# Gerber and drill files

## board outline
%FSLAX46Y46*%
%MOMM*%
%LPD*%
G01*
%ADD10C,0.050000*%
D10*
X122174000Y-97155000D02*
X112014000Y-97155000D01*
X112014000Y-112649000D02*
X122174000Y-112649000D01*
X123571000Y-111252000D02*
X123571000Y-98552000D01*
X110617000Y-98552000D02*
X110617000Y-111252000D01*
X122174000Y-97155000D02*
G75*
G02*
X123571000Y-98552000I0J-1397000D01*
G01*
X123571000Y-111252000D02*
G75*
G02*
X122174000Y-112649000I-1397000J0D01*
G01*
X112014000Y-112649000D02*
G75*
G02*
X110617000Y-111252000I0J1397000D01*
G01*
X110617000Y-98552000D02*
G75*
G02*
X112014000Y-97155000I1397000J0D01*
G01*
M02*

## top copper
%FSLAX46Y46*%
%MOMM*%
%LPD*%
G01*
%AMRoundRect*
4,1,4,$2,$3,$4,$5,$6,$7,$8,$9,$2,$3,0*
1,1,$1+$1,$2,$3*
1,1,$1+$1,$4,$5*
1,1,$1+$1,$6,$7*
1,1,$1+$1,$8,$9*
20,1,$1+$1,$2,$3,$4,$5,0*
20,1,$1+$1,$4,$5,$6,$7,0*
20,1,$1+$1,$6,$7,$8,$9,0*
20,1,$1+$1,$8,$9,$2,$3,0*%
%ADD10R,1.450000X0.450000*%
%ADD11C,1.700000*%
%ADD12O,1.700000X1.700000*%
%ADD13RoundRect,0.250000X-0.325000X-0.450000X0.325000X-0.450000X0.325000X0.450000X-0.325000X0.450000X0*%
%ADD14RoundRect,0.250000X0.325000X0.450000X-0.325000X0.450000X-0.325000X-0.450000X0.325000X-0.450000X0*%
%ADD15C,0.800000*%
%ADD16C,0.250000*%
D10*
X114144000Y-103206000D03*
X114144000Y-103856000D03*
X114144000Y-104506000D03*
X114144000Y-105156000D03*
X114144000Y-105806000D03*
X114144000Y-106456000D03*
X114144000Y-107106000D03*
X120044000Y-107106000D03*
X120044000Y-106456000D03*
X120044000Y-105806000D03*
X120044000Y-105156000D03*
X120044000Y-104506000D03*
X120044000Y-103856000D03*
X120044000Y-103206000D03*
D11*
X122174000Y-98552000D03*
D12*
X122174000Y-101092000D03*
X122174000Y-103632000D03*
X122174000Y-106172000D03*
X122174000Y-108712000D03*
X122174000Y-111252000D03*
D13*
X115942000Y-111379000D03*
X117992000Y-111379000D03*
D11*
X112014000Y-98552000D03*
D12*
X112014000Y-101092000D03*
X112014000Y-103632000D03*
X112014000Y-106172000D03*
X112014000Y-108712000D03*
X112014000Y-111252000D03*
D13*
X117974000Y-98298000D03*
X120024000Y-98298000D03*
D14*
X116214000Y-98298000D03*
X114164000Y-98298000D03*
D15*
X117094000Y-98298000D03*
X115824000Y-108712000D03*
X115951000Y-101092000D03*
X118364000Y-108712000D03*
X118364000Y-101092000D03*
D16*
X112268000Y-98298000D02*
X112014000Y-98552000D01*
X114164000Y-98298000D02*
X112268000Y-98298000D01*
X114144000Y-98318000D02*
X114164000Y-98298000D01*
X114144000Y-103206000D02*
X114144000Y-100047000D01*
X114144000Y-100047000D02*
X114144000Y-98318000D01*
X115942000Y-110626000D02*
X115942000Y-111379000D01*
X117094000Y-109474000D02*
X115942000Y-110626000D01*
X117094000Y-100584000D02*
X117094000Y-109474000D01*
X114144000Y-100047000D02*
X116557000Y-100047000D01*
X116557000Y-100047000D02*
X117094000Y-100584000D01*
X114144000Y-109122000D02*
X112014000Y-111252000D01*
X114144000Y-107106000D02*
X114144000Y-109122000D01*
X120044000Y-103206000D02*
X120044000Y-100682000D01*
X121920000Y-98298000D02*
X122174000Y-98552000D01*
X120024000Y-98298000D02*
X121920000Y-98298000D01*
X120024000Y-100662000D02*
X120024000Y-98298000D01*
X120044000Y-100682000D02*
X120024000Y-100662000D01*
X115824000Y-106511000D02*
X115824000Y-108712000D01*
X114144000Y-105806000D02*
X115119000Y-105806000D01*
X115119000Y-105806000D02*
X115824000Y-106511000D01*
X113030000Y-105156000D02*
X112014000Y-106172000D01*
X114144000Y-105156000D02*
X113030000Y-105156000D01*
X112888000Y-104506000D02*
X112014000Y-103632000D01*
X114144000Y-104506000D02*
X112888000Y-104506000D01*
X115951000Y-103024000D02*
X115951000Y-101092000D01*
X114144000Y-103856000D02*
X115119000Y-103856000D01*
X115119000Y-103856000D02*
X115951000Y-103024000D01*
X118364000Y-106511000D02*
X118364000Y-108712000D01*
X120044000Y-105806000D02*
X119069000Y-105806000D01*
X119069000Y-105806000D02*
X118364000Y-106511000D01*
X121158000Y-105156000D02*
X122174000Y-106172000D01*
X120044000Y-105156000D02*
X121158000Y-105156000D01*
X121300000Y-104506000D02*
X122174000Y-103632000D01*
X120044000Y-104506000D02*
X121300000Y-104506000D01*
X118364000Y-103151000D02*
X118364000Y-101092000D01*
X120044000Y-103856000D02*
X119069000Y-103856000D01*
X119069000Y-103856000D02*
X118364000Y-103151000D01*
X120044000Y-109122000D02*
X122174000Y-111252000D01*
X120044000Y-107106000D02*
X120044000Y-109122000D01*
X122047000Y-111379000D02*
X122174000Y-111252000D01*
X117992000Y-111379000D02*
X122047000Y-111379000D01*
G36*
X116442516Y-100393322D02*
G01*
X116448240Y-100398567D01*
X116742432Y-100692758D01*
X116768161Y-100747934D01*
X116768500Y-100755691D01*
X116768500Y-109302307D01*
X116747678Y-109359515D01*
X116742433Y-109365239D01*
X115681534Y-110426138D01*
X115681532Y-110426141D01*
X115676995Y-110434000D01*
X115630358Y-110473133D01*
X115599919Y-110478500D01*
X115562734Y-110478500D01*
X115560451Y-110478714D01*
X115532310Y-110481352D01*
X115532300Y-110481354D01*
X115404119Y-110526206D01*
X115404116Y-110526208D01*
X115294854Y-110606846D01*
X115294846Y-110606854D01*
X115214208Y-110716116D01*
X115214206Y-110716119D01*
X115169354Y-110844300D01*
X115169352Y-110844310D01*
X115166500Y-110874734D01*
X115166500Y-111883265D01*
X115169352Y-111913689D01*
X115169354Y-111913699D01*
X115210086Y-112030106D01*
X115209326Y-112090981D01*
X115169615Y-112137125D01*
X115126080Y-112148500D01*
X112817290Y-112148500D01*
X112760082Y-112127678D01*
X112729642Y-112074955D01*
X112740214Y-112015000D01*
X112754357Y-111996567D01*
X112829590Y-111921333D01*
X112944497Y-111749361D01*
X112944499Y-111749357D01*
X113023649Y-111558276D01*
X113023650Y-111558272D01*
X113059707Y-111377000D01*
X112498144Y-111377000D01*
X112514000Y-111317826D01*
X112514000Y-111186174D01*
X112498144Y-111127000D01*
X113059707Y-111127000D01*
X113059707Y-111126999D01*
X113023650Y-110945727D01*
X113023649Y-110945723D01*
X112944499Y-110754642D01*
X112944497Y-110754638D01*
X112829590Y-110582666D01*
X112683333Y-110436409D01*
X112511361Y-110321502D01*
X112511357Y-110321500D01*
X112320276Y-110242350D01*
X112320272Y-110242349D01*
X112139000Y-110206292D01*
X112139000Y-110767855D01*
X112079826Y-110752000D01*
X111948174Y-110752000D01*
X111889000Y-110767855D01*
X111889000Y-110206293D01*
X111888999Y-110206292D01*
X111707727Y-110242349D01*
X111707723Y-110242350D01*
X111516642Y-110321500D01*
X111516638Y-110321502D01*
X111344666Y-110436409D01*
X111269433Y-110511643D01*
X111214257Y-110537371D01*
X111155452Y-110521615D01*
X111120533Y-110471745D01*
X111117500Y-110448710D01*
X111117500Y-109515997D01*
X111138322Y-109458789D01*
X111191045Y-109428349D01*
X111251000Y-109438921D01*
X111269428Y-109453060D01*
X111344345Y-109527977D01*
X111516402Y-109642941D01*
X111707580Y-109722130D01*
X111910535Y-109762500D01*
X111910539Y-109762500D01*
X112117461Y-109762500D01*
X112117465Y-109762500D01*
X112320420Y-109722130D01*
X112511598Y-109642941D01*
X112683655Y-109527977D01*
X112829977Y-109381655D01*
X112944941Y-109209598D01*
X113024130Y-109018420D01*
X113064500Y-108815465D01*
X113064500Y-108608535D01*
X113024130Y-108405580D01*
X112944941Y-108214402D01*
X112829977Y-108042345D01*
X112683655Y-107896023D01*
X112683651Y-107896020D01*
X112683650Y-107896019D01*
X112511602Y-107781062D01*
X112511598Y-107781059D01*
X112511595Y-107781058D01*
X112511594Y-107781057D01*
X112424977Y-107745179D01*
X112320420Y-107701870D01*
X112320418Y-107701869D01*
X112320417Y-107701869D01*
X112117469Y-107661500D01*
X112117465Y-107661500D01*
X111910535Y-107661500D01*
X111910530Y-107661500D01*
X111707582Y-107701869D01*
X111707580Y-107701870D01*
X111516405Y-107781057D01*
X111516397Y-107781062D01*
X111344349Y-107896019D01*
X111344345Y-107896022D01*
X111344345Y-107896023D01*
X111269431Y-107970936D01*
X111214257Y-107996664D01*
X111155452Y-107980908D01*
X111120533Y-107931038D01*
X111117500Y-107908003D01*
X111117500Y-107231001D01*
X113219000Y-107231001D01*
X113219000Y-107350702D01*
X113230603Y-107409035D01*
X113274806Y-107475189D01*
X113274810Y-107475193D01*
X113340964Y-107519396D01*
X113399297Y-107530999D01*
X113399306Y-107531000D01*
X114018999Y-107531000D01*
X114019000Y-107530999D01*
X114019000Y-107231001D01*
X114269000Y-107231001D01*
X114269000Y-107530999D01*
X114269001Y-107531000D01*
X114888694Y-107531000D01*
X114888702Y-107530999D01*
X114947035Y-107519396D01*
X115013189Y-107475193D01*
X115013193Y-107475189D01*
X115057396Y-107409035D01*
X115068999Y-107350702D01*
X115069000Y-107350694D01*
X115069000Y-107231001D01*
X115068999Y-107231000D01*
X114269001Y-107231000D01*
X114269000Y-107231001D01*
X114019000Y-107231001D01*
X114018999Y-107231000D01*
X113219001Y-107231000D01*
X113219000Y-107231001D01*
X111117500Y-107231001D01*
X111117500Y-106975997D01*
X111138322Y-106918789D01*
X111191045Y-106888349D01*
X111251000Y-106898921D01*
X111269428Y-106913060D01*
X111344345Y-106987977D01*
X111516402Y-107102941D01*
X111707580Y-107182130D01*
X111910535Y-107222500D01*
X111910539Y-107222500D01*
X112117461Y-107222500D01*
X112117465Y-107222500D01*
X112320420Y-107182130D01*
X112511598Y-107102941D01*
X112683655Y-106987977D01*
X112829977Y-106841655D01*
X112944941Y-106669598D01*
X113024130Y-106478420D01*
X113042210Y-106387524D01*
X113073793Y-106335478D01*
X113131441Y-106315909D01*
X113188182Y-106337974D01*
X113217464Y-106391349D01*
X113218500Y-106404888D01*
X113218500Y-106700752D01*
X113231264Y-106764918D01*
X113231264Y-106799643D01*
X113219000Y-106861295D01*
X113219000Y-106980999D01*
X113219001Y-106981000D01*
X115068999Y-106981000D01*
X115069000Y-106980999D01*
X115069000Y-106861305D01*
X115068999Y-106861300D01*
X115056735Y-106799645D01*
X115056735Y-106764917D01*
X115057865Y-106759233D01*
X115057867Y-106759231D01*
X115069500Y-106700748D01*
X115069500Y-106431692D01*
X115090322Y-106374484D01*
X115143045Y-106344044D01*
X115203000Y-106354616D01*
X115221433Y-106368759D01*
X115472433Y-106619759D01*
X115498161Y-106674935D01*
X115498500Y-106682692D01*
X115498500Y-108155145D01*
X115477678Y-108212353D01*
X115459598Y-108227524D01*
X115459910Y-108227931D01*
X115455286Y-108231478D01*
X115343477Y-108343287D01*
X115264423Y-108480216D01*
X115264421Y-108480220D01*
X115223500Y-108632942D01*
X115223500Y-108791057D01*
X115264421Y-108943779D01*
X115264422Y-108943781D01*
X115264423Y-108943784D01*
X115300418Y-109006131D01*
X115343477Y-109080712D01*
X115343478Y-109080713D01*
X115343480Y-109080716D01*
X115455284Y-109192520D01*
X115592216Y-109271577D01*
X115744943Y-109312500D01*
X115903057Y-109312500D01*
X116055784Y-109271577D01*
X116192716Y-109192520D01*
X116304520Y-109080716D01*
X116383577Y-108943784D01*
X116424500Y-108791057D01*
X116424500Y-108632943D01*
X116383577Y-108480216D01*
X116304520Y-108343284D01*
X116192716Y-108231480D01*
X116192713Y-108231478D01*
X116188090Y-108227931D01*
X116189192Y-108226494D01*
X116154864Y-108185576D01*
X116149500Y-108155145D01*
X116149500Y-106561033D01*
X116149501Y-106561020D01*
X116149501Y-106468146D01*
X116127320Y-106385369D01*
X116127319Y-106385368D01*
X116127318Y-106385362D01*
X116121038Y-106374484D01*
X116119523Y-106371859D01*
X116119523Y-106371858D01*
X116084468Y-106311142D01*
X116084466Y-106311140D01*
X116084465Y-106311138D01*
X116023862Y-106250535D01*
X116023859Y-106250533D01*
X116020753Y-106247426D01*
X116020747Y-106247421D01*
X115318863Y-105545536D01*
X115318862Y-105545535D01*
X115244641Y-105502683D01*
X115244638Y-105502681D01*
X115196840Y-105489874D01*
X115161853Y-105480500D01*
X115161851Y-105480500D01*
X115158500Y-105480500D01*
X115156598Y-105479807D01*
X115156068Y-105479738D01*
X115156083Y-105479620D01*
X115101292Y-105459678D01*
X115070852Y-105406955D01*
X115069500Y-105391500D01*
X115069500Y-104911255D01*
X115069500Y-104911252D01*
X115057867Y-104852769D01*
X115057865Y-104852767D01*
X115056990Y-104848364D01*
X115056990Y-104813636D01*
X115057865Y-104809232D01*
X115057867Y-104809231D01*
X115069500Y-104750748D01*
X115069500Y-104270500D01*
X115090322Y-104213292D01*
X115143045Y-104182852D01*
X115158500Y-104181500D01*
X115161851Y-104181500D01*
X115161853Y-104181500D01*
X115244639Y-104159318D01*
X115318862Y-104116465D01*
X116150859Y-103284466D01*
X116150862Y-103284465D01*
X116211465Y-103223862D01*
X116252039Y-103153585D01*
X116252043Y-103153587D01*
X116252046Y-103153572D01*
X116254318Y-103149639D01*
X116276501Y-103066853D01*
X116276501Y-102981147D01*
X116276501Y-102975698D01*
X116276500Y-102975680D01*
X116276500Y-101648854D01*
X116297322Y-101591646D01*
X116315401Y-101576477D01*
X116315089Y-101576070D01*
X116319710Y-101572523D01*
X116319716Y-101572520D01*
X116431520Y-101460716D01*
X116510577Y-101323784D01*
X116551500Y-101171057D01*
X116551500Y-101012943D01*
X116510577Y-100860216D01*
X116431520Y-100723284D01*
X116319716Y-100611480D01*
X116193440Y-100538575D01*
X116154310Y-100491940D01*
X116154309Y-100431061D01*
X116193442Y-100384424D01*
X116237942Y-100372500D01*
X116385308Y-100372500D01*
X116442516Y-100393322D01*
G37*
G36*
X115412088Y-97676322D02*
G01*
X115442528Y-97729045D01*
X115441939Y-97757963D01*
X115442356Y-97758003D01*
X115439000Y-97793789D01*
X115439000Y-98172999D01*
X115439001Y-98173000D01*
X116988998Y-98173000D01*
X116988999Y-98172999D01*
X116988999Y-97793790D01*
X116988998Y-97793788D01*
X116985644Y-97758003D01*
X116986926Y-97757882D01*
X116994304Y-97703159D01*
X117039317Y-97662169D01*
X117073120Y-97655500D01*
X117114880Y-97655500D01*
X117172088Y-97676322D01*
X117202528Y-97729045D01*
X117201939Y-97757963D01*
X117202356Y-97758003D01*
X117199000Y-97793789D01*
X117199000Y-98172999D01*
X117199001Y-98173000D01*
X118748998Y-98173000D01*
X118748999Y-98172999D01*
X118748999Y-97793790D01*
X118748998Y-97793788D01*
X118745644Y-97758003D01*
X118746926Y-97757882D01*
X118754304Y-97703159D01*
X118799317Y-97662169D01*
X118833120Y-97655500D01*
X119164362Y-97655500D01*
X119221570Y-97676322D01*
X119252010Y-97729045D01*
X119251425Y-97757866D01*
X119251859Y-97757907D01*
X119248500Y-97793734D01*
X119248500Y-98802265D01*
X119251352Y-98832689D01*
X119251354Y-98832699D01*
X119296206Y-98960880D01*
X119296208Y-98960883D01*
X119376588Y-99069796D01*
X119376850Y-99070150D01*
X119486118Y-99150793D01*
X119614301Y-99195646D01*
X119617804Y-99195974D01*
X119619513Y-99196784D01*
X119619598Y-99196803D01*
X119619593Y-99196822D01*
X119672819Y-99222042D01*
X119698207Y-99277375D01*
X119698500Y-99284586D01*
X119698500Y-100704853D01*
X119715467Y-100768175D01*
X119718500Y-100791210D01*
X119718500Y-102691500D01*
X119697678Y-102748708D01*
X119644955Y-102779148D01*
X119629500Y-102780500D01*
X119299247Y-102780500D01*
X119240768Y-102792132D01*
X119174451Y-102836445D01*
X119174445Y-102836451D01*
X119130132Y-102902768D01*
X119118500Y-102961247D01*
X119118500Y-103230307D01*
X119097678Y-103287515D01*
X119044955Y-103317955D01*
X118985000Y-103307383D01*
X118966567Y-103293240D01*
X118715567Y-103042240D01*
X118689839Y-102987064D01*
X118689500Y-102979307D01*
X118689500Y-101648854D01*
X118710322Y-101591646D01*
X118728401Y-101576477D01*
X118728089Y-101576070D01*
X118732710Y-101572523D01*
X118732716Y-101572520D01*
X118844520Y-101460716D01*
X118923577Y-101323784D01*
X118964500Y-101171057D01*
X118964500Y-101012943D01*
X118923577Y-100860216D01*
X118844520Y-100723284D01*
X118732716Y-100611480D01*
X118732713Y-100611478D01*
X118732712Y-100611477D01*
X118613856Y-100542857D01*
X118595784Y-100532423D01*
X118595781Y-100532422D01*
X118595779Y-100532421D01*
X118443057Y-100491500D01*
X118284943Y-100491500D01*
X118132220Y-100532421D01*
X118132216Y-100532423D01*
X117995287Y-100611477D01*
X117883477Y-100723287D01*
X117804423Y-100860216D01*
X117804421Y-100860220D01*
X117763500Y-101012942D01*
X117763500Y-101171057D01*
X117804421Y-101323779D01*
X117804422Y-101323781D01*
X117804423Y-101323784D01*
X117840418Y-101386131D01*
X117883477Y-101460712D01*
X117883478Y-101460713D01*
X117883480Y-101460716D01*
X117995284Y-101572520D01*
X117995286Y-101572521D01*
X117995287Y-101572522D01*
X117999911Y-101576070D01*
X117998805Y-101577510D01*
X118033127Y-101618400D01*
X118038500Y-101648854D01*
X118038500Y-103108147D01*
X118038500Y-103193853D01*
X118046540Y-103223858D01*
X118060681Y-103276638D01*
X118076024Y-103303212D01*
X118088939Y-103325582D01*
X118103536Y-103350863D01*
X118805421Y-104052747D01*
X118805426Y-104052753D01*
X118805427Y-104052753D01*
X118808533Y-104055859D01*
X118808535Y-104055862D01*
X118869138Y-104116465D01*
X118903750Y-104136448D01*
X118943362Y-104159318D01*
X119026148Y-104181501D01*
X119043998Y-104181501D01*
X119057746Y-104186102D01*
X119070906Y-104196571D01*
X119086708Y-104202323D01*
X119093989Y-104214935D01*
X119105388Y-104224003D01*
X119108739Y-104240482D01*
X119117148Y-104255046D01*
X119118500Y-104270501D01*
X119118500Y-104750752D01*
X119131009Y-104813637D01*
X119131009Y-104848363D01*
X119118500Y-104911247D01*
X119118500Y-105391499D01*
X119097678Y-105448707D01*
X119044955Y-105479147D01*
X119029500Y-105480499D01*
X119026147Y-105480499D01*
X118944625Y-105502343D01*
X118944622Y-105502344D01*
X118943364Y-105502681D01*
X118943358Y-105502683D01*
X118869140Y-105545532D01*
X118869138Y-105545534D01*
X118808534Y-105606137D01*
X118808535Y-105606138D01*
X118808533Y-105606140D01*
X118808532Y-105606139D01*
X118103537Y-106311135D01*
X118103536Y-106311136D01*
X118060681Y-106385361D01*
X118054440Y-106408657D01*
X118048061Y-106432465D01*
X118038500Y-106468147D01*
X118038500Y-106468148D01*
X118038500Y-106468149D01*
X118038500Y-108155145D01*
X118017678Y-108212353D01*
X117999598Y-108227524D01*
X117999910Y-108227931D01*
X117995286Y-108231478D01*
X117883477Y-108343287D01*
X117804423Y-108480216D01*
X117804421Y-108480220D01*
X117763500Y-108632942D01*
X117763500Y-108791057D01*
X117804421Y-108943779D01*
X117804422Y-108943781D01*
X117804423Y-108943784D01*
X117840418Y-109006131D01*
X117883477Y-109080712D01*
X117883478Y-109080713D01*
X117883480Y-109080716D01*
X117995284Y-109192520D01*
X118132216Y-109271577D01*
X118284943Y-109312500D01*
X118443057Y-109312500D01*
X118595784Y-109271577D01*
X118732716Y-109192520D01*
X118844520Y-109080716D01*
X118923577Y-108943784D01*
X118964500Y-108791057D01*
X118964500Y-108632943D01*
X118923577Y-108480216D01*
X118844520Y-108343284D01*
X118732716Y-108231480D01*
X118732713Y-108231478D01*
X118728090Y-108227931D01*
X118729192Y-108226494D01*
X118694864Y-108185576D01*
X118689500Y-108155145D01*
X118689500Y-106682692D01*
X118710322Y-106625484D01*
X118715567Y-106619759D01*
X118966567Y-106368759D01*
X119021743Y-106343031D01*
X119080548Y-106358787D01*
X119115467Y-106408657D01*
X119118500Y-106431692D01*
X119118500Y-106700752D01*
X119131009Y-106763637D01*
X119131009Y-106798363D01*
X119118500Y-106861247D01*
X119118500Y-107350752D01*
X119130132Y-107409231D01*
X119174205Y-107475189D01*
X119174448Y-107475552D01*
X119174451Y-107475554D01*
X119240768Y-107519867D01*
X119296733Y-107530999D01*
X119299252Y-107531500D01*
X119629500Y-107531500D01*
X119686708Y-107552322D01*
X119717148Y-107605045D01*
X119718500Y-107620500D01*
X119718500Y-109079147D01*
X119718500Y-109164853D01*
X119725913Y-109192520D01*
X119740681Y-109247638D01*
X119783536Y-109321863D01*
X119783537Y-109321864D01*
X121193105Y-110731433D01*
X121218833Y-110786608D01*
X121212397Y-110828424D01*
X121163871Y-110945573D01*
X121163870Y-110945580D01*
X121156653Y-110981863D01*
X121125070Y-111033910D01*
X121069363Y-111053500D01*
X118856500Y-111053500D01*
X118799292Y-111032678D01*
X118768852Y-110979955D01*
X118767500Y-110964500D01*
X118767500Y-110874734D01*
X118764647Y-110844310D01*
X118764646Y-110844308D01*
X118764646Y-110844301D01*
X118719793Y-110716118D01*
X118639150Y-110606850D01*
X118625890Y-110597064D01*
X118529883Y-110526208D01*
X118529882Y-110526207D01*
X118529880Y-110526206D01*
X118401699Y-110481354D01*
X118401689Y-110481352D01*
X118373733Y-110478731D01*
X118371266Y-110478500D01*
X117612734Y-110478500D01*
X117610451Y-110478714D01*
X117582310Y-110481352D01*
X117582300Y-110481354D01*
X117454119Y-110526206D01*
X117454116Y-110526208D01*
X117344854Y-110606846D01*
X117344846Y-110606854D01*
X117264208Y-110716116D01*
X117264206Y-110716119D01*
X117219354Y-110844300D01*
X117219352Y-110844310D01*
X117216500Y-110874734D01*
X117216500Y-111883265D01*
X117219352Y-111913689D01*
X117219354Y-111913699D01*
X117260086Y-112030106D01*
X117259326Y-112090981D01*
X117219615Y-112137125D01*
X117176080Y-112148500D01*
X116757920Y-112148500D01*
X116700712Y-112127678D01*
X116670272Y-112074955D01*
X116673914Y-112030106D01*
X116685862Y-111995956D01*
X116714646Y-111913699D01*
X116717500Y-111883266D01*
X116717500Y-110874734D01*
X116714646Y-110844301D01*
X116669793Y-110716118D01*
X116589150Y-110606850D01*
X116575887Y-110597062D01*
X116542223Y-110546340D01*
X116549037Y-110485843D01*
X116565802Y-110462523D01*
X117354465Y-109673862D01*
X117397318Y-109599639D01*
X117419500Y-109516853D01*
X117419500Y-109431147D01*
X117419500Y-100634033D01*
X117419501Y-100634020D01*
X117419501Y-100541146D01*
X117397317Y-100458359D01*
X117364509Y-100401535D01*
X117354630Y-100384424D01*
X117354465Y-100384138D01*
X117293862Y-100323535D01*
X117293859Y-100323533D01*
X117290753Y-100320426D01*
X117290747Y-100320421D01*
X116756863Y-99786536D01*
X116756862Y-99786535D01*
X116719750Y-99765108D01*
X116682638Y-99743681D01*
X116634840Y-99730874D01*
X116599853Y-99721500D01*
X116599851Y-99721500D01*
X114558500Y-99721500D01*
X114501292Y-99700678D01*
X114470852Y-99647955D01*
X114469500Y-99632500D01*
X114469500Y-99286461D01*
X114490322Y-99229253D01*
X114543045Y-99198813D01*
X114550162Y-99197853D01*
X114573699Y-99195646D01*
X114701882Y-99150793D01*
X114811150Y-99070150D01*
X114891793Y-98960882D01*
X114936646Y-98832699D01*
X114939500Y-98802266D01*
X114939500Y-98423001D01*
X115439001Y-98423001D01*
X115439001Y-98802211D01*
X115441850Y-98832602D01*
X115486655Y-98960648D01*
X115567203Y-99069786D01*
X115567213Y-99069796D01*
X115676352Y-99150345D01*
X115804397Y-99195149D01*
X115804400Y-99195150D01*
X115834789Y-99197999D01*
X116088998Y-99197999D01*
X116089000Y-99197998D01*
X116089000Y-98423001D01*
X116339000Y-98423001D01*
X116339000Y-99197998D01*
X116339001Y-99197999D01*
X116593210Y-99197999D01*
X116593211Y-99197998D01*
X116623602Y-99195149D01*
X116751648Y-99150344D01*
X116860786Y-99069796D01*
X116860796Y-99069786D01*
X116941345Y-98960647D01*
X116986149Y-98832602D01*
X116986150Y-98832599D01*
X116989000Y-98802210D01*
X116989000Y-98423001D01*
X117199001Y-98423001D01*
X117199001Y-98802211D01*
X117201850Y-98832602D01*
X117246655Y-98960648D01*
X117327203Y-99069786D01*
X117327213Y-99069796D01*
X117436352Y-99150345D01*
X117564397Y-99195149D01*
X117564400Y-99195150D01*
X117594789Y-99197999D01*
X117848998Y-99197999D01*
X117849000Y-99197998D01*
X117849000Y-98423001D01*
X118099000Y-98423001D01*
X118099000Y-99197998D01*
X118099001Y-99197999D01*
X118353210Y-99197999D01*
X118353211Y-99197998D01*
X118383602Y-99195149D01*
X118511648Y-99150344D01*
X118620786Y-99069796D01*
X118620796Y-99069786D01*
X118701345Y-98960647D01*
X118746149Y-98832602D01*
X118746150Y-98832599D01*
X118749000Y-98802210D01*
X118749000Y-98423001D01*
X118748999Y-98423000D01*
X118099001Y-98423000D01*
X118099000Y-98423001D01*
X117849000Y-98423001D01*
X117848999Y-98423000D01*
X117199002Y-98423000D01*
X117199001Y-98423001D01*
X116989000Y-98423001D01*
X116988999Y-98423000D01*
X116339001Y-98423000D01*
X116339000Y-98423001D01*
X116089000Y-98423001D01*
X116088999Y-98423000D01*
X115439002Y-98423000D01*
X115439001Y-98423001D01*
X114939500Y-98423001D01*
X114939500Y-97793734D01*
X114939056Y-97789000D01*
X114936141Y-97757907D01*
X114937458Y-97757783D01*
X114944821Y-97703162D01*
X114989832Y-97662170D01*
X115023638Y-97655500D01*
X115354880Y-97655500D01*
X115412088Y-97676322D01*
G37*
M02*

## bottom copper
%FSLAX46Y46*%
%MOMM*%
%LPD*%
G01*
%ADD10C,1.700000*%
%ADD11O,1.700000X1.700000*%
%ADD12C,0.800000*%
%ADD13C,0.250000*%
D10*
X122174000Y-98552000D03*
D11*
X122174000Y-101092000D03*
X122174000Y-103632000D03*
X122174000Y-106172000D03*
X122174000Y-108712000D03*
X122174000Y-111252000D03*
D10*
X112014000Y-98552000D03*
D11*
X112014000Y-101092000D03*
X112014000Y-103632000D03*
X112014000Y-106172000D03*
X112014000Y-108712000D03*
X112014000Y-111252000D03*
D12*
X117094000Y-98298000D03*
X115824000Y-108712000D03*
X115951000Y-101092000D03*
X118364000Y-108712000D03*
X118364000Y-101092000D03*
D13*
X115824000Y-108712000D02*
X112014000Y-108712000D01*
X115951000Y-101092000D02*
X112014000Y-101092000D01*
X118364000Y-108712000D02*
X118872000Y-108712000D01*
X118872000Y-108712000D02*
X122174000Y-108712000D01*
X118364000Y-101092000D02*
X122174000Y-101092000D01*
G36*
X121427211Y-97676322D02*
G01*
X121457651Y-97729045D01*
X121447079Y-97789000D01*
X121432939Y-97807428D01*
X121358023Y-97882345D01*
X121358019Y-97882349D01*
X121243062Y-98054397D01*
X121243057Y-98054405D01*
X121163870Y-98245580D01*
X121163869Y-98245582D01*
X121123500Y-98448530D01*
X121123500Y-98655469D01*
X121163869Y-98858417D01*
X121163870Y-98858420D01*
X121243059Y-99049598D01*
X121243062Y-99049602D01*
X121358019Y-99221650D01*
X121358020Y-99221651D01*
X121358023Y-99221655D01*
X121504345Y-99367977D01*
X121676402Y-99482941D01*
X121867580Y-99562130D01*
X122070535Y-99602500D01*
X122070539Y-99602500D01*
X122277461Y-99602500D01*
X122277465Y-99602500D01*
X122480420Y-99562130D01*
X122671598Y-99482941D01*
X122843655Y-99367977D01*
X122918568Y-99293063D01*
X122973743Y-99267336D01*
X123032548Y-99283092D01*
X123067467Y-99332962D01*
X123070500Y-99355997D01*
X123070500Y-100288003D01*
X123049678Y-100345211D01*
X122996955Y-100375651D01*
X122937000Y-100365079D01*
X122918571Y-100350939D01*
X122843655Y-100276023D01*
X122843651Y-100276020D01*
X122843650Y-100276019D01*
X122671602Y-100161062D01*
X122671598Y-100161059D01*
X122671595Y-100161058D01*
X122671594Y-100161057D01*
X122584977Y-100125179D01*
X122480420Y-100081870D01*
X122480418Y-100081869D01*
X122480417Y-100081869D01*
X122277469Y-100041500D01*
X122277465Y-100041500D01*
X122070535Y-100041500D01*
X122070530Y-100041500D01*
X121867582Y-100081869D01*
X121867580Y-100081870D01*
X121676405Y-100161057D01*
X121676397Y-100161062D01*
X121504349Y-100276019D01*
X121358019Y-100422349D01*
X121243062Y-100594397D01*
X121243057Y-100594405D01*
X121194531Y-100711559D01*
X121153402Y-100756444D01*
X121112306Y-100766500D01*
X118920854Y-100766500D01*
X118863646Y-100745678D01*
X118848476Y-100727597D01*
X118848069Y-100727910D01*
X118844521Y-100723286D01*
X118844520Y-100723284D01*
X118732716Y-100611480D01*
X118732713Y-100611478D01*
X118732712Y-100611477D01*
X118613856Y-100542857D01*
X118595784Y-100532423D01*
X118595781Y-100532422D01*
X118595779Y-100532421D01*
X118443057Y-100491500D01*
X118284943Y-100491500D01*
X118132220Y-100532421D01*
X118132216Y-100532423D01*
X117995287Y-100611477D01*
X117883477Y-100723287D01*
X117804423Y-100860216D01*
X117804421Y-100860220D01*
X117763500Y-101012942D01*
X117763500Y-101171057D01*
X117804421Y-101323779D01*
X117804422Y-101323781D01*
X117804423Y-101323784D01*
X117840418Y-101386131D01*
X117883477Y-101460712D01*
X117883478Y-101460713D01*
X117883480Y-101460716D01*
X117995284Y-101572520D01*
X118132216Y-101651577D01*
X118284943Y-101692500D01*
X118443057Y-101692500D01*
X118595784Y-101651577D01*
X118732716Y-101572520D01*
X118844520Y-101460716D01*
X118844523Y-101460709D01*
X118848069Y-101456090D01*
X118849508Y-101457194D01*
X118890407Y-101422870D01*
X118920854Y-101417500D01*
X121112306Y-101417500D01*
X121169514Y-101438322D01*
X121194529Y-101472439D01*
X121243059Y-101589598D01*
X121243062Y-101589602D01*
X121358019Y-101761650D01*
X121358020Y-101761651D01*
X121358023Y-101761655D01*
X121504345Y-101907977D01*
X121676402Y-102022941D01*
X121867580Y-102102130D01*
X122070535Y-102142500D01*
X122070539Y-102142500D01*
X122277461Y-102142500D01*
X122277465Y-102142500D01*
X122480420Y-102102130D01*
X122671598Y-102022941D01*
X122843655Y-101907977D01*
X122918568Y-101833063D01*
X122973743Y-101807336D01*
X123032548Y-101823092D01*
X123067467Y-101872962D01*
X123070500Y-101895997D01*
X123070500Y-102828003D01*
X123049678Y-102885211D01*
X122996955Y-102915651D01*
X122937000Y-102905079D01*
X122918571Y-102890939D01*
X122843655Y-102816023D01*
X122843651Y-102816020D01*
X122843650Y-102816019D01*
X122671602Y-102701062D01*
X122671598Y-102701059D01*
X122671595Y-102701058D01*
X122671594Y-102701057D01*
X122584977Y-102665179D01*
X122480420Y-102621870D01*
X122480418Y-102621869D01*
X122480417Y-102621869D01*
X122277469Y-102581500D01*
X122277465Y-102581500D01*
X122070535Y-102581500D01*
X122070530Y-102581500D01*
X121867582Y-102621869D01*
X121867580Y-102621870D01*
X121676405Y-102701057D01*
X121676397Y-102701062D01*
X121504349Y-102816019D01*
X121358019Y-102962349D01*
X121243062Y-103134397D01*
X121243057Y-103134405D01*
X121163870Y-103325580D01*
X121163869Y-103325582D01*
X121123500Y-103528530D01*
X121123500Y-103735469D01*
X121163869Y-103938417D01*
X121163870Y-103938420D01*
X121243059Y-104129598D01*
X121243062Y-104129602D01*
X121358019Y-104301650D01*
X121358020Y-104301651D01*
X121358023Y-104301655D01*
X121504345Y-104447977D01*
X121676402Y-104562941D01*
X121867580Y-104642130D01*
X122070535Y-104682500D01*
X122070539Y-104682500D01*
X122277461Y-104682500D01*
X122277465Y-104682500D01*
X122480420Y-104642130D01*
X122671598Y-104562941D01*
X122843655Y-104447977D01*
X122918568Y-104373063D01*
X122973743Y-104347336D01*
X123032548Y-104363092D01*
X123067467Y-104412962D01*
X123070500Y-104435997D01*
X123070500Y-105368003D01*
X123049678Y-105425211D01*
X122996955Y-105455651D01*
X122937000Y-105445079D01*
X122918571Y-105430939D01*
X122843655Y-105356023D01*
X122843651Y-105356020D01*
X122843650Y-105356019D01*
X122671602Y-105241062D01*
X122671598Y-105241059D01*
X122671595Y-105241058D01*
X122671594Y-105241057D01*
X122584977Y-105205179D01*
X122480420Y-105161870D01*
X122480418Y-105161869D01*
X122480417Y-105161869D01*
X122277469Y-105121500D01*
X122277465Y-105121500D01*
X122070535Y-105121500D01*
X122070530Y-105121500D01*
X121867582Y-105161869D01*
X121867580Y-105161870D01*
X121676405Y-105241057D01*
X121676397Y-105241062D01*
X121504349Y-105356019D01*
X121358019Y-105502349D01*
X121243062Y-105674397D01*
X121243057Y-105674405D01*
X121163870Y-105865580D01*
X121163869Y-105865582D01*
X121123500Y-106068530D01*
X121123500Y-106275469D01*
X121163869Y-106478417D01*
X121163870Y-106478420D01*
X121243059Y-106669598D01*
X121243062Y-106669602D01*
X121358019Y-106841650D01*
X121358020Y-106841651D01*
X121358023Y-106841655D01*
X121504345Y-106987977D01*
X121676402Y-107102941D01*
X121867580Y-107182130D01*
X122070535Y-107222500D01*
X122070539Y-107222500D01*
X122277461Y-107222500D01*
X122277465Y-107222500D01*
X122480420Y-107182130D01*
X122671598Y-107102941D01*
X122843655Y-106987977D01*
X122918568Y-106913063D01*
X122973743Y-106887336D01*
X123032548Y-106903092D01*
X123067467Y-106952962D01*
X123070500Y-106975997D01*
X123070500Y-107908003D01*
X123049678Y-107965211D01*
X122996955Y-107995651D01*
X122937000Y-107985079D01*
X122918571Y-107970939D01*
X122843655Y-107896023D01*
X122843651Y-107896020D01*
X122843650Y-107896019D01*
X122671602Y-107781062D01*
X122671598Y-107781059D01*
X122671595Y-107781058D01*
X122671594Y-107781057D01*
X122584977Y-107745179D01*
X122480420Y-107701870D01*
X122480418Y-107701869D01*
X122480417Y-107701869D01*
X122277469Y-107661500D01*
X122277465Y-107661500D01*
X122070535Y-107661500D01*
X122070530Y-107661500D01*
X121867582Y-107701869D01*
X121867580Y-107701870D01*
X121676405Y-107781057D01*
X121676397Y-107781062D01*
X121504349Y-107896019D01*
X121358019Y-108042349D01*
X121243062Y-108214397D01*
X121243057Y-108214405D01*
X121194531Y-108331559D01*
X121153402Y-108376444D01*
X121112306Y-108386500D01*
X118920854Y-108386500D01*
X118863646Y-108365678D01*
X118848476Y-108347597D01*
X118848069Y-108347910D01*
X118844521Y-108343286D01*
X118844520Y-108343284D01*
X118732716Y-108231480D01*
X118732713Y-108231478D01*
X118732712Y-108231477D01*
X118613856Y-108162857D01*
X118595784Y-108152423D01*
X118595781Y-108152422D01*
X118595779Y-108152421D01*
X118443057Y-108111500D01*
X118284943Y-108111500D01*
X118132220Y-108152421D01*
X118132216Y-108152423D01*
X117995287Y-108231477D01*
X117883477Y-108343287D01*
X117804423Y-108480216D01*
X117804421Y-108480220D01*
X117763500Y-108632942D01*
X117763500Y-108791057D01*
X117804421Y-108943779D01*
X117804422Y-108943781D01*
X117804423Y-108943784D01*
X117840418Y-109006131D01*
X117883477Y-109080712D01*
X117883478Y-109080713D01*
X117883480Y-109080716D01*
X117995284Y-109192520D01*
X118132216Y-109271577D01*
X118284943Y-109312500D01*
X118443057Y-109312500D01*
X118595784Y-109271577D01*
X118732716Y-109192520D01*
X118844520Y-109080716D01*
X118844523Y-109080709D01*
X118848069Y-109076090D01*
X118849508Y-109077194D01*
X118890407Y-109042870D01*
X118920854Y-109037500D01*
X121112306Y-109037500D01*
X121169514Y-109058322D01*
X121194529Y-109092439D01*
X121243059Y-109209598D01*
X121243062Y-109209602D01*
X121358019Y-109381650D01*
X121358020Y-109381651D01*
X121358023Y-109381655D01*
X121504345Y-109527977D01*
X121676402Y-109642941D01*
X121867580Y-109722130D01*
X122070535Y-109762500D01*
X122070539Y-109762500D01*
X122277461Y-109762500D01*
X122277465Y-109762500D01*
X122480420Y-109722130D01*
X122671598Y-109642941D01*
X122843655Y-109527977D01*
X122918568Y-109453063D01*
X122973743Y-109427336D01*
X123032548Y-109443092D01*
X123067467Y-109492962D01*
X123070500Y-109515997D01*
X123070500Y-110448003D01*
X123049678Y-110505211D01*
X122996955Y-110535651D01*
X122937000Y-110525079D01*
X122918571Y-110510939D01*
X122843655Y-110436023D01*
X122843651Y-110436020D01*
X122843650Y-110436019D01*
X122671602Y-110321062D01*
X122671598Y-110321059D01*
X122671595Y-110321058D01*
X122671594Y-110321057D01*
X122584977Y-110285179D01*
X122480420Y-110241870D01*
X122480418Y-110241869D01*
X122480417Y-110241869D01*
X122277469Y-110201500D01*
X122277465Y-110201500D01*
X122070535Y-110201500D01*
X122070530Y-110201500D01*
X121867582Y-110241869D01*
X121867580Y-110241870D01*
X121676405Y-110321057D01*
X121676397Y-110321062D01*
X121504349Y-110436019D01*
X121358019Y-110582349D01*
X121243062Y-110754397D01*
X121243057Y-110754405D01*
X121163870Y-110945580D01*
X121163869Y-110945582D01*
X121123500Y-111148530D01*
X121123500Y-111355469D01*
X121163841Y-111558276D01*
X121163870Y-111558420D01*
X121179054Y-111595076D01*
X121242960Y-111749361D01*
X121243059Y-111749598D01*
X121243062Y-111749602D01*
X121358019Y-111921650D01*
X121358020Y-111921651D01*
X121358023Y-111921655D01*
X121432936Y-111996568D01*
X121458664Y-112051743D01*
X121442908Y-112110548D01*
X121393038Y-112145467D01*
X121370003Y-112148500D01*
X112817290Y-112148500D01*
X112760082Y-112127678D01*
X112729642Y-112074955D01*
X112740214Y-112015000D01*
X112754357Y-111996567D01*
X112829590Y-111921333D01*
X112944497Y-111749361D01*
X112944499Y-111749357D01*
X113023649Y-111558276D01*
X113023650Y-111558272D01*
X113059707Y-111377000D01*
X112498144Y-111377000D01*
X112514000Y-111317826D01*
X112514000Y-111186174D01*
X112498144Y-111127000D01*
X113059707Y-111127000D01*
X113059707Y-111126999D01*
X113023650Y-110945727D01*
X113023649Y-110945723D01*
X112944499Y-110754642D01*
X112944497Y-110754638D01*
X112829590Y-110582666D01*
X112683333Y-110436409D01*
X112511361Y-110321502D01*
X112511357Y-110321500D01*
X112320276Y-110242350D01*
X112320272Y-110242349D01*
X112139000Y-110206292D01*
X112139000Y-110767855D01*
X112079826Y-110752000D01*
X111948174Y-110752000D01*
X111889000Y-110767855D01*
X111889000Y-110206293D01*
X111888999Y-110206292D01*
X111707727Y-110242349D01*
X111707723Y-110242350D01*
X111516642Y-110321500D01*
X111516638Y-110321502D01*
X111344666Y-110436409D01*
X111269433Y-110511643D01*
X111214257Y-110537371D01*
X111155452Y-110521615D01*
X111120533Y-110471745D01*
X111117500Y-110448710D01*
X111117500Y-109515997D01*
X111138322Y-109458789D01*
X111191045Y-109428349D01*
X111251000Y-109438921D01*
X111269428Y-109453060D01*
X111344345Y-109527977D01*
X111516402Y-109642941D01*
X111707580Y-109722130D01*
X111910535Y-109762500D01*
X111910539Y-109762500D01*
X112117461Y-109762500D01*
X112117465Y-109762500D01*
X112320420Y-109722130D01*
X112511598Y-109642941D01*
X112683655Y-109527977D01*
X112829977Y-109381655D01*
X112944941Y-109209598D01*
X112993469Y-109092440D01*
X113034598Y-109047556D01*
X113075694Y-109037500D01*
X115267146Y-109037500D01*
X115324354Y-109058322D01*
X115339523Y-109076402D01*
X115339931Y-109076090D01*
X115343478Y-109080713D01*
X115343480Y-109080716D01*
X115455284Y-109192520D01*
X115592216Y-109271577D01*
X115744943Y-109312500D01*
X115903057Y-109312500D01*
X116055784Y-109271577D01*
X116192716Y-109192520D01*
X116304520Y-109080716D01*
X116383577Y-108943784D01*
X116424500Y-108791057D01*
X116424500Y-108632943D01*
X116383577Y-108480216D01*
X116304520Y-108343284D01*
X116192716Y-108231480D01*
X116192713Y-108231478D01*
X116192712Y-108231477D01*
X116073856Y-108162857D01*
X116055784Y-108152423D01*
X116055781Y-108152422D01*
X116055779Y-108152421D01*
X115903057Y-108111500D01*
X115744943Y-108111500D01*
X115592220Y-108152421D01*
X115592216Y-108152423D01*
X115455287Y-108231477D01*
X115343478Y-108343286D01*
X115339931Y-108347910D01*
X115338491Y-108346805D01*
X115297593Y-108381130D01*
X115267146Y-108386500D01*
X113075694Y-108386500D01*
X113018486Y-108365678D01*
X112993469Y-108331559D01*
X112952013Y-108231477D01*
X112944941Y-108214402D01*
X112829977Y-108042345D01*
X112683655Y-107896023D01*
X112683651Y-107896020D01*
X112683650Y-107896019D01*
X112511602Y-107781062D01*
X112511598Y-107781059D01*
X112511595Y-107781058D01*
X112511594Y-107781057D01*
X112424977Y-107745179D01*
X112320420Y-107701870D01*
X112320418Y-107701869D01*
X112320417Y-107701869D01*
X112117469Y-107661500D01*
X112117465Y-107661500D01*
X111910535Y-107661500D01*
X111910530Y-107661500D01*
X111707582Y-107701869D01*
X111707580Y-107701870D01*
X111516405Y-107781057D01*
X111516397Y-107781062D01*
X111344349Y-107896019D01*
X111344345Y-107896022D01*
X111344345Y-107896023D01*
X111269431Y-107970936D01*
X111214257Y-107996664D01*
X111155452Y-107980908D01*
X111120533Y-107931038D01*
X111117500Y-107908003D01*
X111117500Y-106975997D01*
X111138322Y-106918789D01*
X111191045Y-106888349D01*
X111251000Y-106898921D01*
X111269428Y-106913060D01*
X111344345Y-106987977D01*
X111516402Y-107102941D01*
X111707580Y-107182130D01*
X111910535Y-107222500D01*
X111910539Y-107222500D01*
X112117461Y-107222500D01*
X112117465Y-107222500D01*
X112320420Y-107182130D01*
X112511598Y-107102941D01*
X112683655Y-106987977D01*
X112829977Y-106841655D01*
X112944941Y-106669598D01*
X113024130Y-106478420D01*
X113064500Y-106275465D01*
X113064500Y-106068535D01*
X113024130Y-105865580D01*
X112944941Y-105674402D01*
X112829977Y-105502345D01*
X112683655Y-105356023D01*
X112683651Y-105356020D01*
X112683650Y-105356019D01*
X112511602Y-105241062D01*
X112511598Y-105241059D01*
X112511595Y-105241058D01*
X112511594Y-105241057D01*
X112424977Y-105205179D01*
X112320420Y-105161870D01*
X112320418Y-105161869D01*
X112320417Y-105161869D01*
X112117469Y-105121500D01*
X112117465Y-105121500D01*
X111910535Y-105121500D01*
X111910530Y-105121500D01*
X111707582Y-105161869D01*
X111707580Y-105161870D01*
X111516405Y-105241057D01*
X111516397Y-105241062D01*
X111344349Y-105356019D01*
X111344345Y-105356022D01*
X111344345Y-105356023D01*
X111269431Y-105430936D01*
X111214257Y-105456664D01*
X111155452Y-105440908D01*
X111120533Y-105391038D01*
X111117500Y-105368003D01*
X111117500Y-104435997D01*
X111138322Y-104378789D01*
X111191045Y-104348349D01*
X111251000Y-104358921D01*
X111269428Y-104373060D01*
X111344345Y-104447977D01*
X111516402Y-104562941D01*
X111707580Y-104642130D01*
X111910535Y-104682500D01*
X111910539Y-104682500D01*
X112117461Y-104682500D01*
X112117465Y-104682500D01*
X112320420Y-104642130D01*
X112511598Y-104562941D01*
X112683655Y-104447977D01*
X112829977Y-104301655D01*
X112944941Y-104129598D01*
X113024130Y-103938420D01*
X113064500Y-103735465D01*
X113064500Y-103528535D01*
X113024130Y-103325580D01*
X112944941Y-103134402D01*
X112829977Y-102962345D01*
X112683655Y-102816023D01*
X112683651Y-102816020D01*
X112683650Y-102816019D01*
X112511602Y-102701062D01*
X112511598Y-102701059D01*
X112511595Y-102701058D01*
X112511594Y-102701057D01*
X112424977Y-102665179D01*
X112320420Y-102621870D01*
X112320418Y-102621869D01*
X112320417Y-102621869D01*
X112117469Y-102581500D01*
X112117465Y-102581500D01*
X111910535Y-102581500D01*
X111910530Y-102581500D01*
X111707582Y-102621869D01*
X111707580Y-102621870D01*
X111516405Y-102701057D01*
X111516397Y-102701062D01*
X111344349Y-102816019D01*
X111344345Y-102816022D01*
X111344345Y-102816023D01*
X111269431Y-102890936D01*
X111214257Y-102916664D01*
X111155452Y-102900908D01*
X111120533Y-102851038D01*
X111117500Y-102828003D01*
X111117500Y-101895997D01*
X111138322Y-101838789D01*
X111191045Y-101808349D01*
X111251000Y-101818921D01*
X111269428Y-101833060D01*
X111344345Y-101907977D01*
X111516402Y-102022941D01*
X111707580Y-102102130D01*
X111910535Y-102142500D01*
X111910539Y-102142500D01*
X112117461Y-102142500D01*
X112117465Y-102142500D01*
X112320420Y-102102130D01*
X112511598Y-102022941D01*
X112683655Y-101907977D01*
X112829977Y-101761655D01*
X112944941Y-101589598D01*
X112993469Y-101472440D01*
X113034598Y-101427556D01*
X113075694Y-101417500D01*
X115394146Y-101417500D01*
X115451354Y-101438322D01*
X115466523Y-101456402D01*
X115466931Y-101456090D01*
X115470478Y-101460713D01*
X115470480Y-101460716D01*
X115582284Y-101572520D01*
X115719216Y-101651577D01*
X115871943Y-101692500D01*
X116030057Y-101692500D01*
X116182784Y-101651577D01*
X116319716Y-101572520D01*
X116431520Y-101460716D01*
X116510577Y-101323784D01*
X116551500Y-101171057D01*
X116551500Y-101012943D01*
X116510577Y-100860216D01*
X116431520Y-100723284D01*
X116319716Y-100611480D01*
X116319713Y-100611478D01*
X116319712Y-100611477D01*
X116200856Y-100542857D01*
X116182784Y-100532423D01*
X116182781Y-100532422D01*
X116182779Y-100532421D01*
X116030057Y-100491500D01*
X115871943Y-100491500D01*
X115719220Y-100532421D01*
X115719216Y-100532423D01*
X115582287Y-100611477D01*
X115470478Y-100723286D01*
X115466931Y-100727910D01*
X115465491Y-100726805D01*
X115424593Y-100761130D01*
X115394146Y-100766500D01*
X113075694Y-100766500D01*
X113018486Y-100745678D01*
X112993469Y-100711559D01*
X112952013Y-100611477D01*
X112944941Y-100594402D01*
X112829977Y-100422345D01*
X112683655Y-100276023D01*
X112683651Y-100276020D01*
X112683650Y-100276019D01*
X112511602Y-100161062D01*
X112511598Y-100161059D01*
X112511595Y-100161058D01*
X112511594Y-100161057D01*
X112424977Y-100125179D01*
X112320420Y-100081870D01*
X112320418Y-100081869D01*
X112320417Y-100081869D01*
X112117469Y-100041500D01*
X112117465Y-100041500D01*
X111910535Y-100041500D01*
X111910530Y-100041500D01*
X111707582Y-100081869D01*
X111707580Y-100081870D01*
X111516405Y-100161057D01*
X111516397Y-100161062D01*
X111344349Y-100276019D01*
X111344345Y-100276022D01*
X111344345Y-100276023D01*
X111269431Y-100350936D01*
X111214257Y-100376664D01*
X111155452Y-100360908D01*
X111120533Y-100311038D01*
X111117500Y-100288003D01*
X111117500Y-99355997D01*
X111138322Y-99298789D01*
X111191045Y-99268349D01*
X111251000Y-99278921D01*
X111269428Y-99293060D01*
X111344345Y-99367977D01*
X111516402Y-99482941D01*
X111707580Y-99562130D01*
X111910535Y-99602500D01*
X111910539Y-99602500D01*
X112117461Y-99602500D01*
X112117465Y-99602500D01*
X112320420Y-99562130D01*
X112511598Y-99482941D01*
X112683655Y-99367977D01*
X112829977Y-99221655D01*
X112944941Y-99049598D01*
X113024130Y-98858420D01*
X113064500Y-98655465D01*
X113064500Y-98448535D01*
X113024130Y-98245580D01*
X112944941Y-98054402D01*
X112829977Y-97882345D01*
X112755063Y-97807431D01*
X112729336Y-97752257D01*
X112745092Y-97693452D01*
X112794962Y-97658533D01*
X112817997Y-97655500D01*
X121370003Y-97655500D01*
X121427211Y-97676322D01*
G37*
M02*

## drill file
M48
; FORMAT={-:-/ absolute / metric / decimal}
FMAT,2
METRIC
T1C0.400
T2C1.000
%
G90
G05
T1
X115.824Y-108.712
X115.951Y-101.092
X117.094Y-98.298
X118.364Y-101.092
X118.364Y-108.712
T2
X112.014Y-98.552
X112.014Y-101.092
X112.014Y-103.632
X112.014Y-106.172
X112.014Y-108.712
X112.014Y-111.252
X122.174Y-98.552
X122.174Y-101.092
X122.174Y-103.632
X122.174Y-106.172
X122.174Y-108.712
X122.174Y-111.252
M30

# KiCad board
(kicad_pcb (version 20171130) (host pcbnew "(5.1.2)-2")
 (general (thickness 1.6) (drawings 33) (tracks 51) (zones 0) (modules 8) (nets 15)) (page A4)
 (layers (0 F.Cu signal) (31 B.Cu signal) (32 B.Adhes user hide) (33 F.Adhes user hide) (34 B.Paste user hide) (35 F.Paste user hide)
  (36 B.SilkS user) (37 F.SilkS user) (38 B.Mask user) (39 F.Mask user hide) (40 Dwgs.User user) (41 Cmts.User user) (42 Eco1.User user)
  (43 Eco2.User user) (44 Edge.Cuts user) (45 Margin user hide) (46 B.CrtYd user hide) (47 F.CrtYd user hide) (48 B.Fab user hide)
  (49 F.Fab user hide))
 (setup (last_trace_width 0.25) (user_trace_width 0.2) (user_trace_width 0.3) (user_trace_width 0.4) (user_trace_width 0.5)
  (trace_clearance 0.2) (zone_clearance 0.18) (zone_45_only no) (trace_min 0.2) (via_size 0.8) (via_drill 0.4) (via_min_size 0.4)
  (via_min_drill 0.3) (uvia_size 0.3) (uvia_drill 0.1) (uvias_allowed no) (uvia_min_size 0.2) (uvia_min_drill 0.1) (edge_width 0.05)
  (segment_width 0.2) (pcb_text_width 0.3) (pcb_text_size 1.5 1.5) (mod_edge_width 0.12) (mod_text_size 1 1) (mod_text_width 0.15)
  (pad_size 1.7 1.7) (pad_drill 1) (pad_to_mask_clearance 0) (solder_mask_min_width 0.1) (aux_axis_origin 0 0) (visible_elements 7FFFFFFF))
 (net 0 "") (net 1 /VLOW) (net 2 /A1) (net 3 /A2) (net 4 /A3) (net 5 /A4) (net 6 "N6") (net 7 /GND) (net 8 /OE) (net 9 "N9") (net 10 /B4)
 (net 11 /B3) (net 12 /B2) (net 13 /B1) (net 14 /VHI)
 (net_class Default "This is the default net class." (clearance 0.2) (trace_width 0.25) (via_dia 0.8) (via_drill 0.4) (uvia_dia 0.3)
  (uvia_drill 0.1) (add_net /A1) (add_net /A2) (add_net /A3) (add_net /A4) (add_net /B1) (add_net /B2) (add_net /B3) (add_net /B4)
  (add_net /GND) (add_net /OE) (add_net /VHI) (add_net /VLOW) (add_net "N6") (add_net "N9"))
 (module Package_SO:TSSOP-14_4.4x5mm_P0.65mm (layer F.Cu) (at 117.094 105.156)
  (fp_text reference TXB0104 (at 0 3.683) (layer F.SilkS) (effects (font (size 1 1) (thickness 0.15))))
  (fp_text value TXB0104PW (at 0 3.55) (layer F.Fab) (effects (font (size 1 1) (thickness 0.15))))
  (pad 1 smd rect (at -2.95 -1.95) (size 1.45 0.45) (layers F.Cu F.Paste F.Mask) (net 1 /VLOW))
  (pad 2 smd rect (at -2.95 -1.3) (size 1.45 0.45) (layers F.Cu F.Paste F.Mask) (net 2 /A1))
  (pad 3 smd rect (at -2.95 -0.65) (size 1.45 0.45) (layers F.Cu F.Paste F.Mask) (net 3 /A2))
  (pad 4 smd rect (at -2.95 0) (size 1.45 0.45) (layers F.Cu F.Paste F.Mask) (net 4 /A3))
  (pad 5 smd rect (at -2.95 0.65) (size 1.45 0.45) (layers F.Cu F.Paste F.Mask) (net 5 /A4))
  (pad 6 smd rect (at -2.95 1.3) (size 1.45 0.45) (layers F.Cu F.Paste F.Mask) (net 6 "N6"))
  (pad 7 smd rect (at -2.95 1.95) (size 1.45 0.45) (layers F.Cu F.Paste F.Mask) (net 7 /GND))
  (pad 8 smd rect (at 2.95 1.95) (size 1.45 0.45) (layers F.Cu F.Paste F.Mask) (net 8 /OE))
  (pad 9 smd rect (at 2.95 1.3) (size 1.45 0.45) (layers F.Cu F.Paste F.Mask) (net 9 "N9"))
  (pad 10 smd rect (at 2.95 0.65) (size 1.45 0.45) (layers F.Cu F.Paste F.Mask) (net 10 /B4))
  (pad 11 smd rect (at 2.95 0) (size 1.45 0.45) (layers F.Cu F.Paste F.Mask) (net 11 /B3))
  (pad 12 smd rect (at 2.95 -0.65) (size 1.45 0.45) (layers F.Cu F.Paste F.Mask) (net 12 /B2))
  (pad 13 smd rect (at 2.95 -1.3) (size 1.45 0.45) (layers F.Cu F.Paste F.Mask) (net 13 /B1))
  (pad 14 smd rect (at 2.95 -1.95) (size 1.45 0.45) (layers F.Cu F.Paste F.Mask) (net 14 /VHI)))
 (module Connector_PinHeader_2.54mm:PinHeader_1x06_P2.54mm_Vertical (layer F.Cu) (at 122.174 98.552)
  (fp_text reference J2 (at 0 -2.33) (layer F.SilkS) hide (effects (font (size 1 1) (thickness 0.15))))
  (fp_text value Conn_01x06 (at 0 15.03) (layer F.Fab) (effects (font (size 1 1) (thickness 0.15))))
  (pad 1 thru_hole circle (at 0 0) (size 1.7 1.7) (drill 1) (layers *.Cu *.Mask) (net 14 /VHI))
  (pad 2 thru_hole oval (at 0 2.54) (size 1.7 1.7) (drill 1) (layers *.Cu *.Mask) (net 13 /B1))
  (pad 3 thru_hole oval (at 0 5.08) (size 1.7 1.7) (drill 1) (layers *.Cu *.Mask) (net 12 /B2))
  (pad 4 thru_hole oval (at 0 7.62) (size 1.7 1.7) (drill 1) (layers *.Cu *.Mask) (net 11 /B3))
  (pad 5 thru_hole oval (at 0 10.16) (size 1.7 1.7) (drill 1) (layers *.Cu *.Mask) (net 10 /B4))
  (pad 6 thru_hole oval (at 0 12.7) (size 1.7 1.7) (drill 1) (layers *.Cu *.Mask) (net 8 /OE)))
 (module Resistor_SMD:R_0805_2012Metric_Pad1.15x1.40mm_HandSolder (layer F.Cu) (at 116.967 111.379)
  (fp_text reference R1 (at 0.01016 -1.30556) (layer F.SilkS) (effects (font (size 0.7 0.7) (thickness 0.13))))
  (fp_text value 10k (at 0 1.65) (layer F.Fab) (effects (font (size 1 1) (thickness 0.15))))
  (pad 1 smd roundrect (at -1.025 0) (size 1.15 1.4) (layers F.Cu F.Paste F.Mask) (roundrect_rratio 0.217391) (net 1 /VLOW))
  (pad 2 smd roundrect (at 1.025 0) (size 1.15 1.4) (layers F.Cu F.Paste F.Mask) (roundrect_rratio 0.217391) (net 8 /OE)))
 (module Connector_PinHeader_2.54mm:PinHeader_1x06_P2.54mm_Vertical (layer F.Cu) (at 112.014 98.552)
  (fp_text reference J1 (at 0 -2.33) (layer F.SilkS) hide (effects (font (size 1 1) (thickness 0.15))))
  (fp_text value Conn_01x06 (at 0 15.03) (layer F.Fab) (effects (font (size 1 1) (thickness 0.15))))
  (pad 1 thru_hole circle (at 0 0) (size 1.7 1.7) (drill 1) (layers *.Cu *.Mask) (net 1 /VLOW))
  (pad 2 thru_hole oval (at 0 2.54) (size 1.7 1.7) (drill 1) (layers *.Cu *.Mask) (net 2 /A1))
  (pad 3 thru_hole oval (at 0 5.08) (size 1.7 1.7) (drill 1) (layers *.Cu *.Mask) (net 3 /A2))
  (pad 4 thru_hole oval (at 0 7.62) (size 1.7 1.7) (drill 1) (layers *.Cu *.Mask) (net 4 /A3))
  (pad 5 thru_hole oval (at 0 10.16) (size 1.7 1.7) (drill 1) (layers *.Cu *.Mask) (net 5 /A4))
  (pad 6 thru_hole oval (at 0 12.7) (size 1.7 1.7) (drill 1) (layers *.Cu *.Mask) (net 7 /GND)))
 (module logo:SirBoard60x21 (layer B.Cu) (at 117.094 102.743 180)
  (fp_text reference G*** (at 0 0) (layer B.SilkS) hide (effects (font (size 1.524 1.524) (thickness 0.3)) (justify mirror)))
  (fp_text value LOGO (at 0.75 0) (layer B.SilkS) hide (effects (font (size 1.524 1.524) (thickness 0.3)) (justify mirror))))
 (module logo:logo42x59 (layer B.Cu) (at 117.094 99.441 180)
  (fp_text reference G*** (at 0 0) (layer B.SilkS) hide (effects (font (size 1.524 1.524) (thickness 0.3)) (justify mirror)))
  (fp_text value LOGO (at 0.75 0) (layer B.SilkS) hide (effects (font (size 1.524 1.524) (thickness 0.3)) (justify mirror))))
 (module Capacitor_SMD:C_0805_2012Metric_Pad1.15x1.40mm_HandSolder (layer F.Cu) (at 118.999 98.298)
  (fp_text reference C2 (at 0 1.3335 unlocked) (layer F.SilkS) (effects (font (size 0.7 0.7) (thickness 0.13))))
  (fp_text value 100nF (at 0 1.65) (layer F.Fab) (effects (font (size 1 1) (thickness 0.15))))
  (pad 1 smd roundrect (at -1.025 0) (size 1.15 1.4) (layers F.Cu F.Paste F.Mask) (roundrect_rratio 0.217391) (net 7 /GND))
  (pad 2 smd roundrect (at 1.025 0) (size 1.15 1.4) (layers F.Cu F.Paste F.Mask) (roundrect_rratio 0.217391) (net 14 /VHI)))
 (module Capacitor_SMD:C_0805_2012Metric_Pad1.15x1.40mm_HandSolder (layer F.Cu) (at 115.189 98.298 180)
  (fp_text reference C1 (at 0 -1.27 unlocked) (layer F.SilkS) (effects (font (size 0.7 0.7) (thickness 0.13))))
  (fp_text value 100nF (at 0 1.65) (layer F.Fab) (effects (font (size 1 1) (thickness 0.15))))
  (pad 1 smd roundrect (at -1.025 0 180) (size 1.15 1.4) (layers F.Cu F.Paste F.Mask) (roundrect_rratio 0.217391) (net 7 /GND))
  (pad 2 smd roundrect (at 1.025 0 180) (size 1.15 1.4) (layers F.Cu F.Paste F.Mask) (roundrect_rratio 0.217391) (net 1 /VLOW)))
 (gr_line (start 122.174 97.155) (end 112.014 97.155) (layer Edge.Cuts) (width 0.05))
 (gr_line (start 112.014 112.649) (end 122.174 112.649) (layer Edge.Cuts) (width 0.05))
 (gr_line (start 123.571 111.252) (end 123.571 98.552) (layer Edge.Cuts) (width 0.05))
 (gr_line (start 110.617 98.552) (end 110.617 111.252) (layer Edge.Cuts) (width 0.05))
 (gr_arc (start 122.174 98.552) (end 123.571 98.552) (angle -90) (layer Edge.Cuts) (width 0.05))
 (gr_arc (start 122.174 111.252) (end 122.174 112.649) (angle -90) (layer Edge.Cuts) (width 0.05))
 (gr_arc (start 112.014 111.252) (end 110.617 111.252) (angle -90) (layer Edge.Cuts) (width 0.05))
 (gr_arc (start 112.014 98.552) (end 112.014 97.155) (angle -90) (layer Edge.Cuts) (width 0.05))
 (segment (start 112.268 98.298) (end 112.014 98.552) (width 0.25) (layer F.Cu) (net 1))
 (segment (start 114.164 98.298) (end 112.268 98.298) (width 0.25) (layer F.Cu) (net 1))
 (segment (start 114.144 98.318) (end 114.164 98.298) (width 0.25) (layer F.Cu) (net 1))
 (segment (start 114.144 103.206) (end 114.144 100.047) (width 0.25) (layer F.Cu) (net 1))
 (segment (start 114.144 100.047) (end 114.144 98.318) (width 0.25) (layer F.Cu) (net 1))
 (segment (start 115.942 110.626) (end 115.942 111.379) (width 0.25) (layer F.Cu) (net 1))
 (segment (start 117.094 109.474) (end 115.942 110.626) (width 0.25) (layer F.Cu) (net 1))
 (segment (start 117.094 100.584) (end 117.094 109.474) (width 0.25) (layer F.Cu) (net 1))
 (segment (start 114.144 100.047) (end 116.557 100.047) (width 0.25) (layer F.Cu) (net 1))
 (segment (start 116.557 100.047) (end 117.094 100.584) (width 0.25) (layer F.Cu) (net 1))
 (segment (start 114.144 109.122) (end 112.014 111.252) (width 0.25) (layer F.Cu) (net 7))
 (segment (start 114.144 107.106) (end 114.144 109.122) (width 0.25) (layer F.Cu) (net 7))
 (via (at 117.094 98.298) (size 0.8) (drill 0.4) (layers F.Cu B.Cu) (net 7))
 (segment (start 120.044 103.206) (end 120.044 100.682) (width 0.25) (layer F.Cu) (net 14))
 (segment (start 121.92 98.298) (end 122.174 98.552) (width 0.25) (layer F.Cu) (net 14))
 (segment (start 120.024 98.298) (end 121.92 98.298) (width 0.25) (layer F.Cu) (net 14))
 (segment (start 120.024 100.662) (end 120.024 98.298) (width 0.25) (layer F.Cu) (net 14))
 (segment (start 120.044 100.682) (end 120.024 100.662) (width 0.25) (layer F.Cu) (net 14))
 (via (at 115.824 108.712) (size 0.8) (drill 0.4) (layers F.Cu B.Cu) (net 5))
 (segment (start 115.824 106.511) (end 115.824 108.712) (width 0.25) (layer F.Cu) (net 5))
 (segment (start 114.144 105.806) (end 115.119 105.806) (width 0.25) (layer F.Cu) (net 5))
 (segment (start 115.119 105.806) (end 115.824 106.511) (width 0.25) (layer F.Cu) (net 5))
 (segment (start 115.824 108.712) (end 112.014 108.712) (width 0.25) (layer B.Cu) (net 5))
 (segment (start 113.03 105.156) (end 112.014 106.172) (width 0.25) (layer F.Cu) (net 4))
 (segment (start 114.144 105.156) (end 113.03 105.156) (width 0.25) (layer F.Cu) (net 4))
 (segment (start 112.888 104.506) (end 112.014 103.632) (width 0.25) (layer F.Cu) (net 3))
 (segment (start 114.144 104.506) (end 112.888 104.506) (width 0.25) (layer F.Cu) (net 3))
 (via (at 115.951 101.092) (size 0.8) (drill 0.4) (layers F.Cu B.Cu) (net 2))
 (segment (start 115.951 103.024) (end 115.951 101.092) (width 0.25) (layer F.Cu) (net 2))
 (segment (start 114.144 103.856) (end 115.119 103.856) (width 0.25) (layer F.Cu) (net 2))
 (segment (start 115.119 103.856) (end 115.951 103.024) (width 0.25) (layer F.Cu) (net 2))
 (segment (start 115.951 101.092) (end 112.014 101.092) (width 0.25) (layer B.Cu) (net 2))
 (via (at 118.364 108.712) (size 0.8) (drill 0.4) (layers F.Cu B.Cu) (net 10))
 (segment (start 118.364 106.511) (end 118.364 108.712) (width 0.25) (layer F.Cu) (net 10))
 (segment (start 120.044 105.806) (end 119.069 105.806) (width 0.25) (layer F.Cu) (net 10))
 (segment (start 119.069 105.806) (end 118.364 106.511) (width 0.25) (layer F.Cu) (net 10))
 (segment (start 118.364 108.712) (end 118.872 108.712) (width 0.25) (layer B.Cu) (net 10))
 (segment (start 118.872 108.712) (end 122.174 108.712) (width 0.25) (layer B.Cu) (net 10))
 (segment (start 121.158 105.156) (end 122.174 106.172) (width 0.25) (layer F.Cu) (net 11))
 (segment (start 120.044 105.156) (end 121.158 105.156) (width 0.25) (layer F.Cu) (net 11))
 (segment (start 121.3 104.506) (end 122.174 103.632) (width 0.25) (layer F.Cu) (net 12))
 (segment (start 120.044 104.506) (end 121.3 104.506) (width 0.25) (layer F.Cu) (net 12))
 (via (at 118.364 101.092) (size 0.8) (drill 0.4) (layers F.Cu B.Cu) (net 13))
 (segment (start 118.364 103.151) (end 118.364 101.092) (width 0.25) (layer F.Cu) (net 13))
 (segment (start 120.044 103.856) (end 119.069 103.856) (width 0.25) (layer F.Cu) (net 13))
 (segment (start 119.069 103.856) (end 118.364 103.151) (width 0.25) (layer F.Cu) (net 13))
 (segment (start 118.364 101.092) (end 122.174 101.092) (width 0.25) (layer B.Cu) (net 13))
 (segment (start 120.044 109.122) (end 122.174 111.252) (width 0.25) (layer F.Cu) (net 8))
 (segment (start 120.044 107.106) (end 120.044 109.122) (width 0.25) (layer F.Cu) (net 8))
 (segment (start 122.047 111.379) (end 122.174 111.252) (width 0.25) (layer F.Cu) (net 8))
 (segment (start 117.992 111.379) (end 122.047 111.379) (width 0.25) (layer F.Cu) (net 8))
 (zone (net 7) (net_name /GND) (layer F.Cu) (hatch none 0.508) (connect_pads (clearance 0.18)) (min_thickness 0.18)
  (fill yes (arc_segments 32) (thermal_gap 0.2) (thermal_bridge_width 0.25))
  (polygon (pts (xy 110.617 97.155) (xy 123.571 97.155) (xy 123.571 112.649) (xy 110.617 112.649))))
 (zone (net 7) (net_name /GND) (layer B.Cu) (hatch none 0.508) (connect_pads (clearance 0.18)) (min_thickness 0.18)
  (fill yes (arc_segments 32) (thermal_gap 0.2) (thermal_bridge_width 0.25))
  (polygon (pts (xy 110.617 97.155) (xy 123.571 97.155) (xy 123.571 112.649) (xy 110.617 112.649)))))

